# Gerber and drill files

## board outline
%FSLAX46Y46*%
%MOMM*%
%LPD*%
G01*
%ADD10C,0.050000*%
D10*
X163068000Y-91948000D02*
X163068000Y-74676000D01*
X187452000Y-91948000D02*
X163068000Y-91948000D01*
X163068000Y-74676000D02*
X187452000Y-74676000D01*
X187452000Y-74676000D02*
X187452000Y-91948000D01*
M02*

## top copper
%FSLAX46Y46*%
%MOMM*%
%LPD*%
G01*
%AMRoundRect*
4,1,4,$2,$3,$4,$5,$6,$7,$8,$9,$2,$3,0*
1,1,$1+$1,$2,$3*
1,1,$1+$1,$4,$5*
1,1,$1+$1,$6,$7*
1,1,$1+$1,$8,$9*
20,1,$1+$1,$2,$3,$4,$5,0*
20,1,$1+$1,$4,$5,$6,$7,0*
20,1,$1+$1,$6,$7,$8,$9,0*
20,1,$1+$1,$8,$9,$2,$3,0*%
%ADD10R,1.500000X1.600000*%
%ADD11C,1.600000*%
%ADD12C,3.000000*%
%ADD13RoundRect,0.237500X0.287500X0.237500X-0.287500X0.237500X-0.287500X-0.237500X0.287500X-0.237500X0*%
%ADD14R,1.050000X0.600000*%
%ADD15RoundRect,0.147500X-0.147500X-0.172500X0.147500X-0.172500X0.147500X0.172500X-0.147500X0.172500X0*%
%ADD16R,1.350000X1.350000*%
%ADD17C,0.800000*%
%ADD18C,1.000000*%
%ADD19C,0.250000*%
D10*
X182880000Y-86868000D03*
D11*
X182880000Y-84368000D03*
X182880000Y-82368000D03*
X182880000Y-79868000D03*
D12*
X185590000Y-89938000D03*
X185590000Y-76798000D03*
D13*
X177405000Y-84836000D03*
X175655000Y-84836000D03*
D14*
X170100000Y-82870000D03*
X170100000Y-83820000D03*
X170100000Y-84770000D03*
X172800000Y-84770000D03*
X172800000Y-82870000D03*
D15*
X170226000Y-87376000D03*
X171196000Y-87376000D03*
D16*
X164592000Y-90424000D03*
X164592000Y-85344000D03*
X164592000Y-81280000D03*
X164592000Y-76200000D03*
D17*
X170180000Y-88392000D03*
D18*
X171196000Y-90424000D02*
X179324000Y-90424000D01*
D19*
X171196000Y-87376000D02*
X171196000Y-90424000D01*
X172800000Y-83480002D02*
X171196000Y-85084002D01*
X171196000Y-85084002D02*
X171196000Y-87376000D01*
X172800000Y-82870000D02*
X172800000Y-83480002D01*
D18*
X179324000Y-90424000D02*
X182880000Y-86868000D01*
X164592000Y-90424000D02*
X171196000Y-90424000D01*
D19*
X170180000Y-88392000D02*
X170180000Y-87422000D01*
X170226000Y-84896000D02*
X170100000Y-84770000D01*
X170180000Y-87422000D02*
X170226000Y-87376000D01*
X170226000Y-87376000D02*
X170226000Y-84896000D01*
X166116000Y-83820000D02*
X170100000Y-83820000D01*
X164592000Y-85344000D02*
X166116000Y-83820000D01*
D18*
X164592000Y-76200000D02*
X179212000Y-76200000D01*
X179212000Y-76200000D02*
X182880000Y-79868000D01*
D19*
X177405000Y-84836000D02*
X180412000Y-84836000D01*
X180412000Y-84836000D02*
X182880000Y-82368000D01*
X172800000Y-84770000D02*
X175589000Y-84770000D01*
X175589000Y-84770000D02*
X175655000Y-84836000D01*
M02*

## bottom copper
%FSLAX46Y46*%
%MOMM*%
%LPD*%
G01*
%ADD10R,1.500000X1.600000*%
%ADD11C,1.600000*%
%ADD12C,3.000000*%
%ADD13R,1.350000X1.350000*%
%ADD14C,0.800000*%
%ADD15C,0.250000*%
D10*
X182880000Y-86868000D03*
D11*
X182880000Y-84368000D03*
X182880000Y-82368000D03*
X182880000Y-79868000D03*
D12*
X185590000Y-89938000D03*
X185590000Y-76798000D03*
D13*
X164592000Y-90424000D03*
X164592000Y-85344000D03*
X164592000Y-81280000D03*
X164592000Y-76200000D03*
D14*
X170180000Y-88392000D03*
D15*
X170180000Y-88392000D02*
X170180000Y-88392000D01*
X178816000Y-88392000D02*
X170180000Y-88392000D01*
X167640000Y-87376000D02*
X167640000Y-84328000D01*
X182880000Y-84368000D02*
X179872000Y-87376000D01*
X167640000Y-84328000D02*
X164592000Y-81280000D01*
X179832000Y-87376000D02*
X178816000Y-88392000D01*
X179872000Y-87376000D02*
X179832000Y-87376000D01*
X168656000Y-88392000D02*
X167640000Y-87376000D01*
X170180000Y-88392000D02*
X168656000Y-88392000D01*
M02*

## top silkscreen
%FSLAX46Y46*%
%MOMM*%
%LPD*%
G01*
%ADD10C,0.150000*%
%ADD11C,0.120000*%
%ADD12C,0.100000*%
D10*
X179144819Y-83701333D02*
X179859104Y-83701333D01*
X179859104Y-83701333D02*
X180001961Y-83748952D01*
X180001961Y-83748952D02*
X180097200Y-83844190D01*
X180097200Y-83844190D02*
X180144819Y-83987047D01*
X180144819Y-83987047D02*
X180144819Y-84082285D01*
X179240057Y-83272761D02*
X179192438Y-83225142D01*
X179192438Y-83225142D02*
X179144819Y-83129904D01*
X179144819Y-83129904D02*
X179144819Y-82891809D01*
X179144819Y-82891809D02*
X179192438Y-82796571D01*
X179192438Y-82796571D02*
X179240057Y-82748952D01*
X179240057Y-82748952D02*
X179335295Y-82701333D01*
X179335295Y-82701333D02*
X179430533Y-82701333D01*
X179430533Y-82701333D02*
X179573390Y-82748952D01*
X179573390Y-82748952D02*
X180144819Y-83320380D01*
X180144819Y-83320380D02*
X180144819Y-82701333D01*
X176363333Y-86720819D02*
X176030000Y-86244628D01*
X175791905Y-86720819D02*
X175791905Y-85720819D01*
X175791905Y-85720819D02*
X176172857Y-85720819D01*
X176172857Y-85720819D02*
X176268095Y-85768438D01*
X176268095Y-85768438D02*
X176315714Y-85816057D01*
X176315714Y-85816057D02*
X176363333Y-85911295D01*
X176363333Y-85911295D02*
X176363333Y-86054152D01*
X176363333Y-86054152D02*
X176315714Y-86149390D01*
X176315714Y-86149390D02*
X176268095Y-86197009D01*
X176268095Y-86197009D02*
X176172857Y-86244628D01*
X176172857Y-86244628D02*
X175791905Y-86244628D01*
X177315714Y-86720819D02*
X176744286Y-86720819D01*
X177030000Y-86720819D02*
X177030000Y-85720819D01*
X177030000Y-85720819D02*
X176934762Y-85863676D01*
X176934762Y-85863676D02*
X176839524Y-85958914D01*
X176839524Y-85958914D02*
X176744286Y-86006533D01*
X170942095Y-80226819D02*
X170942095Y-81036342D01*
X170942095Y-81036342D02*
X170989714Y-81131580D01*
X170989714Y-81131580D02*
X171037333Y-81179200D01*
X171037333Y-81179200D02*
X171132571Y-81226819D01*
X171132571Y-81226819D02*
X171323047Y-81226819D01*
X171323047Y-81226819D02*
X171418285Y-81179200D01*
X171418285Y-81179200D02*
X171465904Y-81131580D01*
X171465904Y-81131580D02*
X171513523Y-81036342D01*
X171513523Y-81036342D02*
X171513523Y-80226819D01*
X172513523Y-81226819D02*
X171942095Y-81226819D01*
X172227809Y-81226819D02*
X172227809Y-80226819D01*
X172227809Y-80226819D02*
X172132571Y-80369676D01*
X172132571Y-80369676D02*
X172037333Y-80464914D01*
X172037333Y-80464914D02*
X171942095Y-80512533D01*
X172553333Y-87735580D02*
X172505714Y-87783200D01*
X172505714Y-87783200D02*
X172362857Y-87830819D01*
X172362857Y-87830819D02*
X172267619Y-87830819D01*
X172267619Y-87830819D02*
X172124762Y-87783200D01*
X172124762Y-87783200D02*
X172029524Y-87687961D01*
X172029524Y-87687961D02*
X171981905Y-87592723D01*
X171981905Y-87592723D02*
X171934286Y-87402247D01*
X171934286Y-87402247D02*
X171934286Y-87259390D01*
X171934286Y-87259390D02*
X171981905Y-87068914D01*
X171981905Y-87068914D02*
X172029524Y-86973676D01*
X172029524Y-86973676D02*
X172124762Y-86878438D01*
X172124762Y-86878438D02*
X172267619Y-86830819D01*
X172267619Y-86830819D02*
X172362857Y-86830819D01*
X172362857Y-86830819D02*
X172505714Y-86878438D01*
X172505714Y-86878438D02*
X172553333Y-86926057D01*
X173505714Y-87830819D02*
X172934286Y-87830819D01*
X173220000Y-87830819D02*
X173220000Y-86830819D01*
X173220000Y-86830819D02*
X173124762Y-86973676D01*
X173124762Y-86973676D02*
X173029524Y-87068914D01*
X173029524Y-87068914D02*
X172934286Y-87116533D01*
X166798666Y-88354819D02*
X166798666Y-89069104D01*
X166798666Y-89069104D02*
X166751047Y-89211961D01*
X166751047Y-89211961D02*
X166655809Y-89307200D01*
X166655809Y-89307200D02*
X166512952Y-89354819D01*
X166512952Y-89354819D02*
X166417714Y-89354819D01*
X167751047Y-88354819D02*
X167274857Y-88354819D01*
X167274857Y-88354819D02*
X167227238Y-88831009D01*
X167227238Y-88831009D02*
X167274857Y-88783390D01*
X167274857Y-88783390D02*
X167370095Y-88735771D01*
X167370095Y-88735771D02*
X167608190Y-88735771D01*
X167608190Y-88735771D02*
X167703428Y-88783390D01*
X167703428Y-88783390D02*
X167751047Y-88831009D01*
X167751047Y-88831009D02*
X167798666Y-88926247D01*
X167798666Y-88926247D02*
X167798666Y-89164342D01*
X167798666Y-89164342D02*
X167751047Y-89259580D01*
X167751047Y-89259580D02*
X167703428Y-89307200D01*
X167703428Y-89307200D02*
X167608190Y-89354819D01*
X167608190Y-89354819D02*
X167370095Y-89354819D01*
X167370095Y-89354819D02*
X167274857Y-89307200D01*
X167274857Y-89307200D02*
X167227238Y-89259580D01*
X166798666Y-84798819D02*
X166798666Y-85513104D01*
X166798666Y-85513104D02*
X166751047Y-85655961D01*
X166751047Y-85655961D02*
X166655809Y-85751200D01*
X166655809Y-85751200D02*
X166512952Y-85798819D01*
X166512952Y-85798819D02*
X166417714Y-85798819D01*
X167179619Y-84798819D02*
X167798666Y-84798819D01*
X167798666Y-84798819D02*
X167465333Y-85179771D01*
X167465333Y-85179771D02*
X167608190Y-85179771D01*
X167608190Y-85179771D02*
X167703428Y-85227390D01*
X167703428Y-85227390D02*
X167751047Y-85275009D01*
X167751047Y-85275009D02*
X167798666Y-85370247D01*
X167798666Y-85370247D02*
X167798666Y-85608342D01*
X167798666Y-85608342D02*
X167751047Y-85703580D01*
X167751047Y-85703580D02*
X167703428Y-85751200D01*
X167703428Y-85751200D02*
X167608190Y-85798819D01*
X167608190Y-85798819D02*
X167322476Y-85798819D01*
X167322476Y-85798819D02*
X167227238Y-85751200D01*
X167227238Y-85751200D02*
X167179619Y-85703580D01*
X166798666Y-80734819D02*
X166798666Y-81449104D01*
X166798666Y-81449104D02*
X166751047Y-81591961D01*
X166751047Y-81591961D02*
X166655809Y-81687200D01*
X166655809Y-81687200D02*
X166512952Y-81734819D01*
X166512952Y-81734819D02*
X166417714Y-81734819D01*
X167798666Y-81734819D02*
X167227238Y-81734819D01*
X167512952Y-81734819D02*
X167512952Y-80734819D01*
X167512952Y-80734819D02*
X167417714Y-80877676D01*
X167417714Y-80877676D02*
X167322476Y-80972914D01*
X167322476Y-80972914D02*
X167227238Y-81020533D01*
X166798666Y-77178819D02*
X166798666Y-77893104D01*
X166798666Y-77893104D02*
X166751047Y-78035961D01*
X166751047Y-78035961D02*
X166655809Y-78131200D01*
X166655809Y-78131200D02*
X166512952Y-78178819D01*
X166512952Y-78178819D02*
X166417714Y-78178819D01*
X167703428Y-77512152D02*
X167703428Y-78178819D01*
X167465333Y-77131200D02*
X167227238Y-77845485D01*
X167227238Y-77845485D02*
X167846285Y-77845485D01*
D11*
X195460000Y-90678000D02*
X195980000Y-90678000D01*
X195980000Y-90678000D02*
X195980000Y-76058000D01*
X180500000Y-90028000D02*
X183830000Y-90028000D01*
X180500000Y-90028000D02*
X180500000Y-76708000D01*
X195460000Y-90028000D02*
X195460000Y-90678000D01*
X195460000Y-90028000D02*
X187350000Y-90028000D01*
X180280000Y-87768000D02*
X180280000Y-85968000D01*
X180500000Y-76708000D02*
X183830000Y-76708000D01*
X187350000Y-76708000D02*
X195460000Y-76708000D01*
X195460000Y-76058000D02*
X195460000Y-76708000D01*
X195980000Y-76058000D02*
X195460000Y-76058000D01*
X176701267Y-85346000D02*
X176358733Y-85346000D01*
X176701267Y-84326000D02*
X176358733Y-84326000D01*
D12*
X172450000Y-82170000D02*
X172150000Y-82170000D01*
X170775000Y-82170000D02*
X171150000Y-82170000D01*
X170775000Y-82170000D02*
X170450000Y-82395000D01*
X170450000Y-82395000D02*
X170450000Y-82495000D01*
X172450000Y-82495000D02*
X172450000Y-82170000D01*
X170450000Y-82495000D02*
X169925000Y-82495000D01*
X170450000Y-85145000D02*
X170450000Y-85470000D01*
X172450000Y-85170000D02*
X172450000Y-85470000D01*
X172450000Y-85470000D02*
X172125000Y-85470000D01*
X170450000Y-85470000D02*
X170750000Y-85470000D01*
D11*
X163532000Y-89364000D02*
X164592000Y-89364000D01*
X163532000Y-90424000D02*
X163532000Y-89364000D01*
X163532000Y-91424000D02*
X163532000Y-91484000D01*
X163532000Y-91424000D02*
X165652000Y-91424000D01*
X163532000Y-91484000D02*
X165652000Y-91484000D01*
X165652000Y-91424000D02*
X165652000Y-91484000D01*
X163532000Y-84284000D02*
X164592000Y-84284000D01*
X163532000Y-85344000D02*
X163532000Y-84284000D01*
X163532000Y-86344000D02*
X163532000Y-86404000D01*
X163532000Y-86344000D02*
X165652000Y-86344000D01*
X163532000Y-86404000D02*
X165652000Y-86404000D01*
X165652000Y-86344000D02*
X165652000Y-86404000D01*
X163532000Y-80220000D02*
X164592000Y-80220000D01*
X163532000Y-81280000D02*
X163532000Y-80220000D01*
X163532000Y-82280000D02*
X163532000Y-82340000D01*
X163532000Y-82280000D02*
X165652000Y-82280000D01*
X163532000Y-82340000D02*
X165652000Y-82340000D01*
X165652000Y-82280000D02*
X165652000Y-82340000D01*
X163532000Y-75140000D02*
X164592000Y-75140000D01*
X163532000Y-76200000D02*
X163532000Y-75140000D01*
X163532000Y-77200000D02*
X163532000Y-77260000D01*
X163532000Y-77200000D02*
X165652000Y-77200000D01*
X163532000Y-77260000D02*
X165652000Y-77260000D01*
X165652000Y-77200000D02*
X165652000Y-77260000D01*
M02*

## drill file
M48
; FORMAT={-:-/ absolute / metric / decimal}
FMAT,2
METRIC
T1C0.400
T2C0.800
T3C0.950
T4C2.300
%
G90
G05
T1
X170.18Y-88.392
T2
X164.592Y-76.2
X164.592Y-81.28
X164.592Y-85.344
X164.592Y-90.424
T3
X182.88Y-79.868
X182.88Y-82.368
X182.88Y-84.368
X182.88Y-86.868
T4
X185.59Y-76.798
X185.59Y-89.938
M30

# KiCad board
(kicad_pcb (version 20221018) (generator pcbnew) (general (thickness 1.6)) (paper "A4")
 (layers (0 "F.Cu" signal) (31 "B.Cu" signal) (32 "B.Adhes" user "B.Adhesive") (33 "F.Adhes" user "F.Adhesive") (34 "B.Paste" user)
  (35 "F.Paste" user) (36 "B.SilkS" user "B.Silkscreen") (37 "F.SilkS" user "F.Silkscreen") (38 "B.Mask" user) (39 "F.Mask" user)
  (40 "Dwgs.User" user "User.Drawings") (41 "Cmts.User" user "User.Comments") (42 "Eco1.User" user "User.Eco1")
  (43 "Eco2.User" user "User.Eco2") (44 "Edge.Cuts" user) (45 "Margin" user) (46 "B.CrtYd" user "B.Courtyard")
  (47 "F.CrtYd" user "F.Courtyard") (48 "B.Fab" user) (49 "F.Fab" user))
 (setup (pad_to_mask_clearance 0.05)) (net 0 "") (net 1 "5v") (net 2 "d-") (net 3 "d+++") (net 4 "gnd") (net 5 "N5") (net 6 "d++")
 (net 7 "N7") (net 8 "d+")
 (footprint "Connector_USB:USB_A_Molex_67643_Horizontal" (layer "F.Cu") (at 182.88 86.868 90)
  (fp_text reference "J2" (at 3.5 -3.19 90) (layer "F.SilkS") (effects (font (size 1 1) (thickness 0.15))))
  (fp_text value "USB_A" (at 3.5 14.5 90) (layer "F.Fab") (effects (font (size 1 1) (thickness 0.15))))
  (fp_line (start -3.81 12.58) (end -3.81 13.1) (stroke (width 0.12) (type solid)) (layer "F.SilkS"))
  (fp_line (start -3.81 13.1) (end 10.81 13.1) (stroke (width 0.12) (type solid)) (layer "F.SilkS"))
  (fp_line (start -3.16 -2.38) (end -3.16 0.95) (stroke (width 0.12) (type solid)) (layer "F.SilkS"))
  (fp_line (start -3.16 -2.38) (end 10.16 -2.38) (stroke (width 0.12) (type solid)) (layer "F.SilkS"))
  (fp_line (start -3.16 12.58) (end -3.81 12.58) (stroke (width 0.12) (type solid)) (layer "F.SilkS"))
  (fp_line (start -3.16 12.58) (end -3.16 4.47) (stroke (width 0.12) (type solid)) (layer "F.SilkS"))
  (fp_line (start -0.9 -2.6) (end 0.9 -2.6) (stroke (width 0.12) (type solid)) (layer "F.SilkS"))
  (fp_line (start 10.16 -2.38) (end 10.16 0.95) (stroke (width 0.12) (type solid)) (layer "F.SilkS"))
  (fp_line (start 10.16 4.47) (end 10.16 12.58) (stroke (width 0.12) (type solid)) (layer "F.SilkS"))
  (fp_line (start 10.81 12.58) (end 10.16 12.58) (stroke (width 0.12) (type solid)) (layer "F.SilkS"))
  (fp_line (start 10.81 13.1) (end 10.81 12.58) (stroke (width 0.12) (type solid)) (layer "F.SilkS"))
  (pad "1" thru_hole rect (at 0 0 90) (size 1.6 1.5) (drill 0.95) (layers "*.Cu" "*.Mask") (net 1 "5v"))
  (pad "2" thru_hole circle (at 2.5 0 90) (size 1.6 1.6) (drill 0.95) (layers "*.Cu" "*.Mask") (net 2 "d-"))
  (pad "3" thru_hole circle (at 4.5 0 90) (size 1.6 1.6) (drill 0.95) (layers "*.Cu" "*.Mask") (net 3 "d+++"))
  (pad "4" thru_hole circle (at 7 0 90) (size 1.6 1.6) (drill 0.95) (layers "*.Cu" "*.Mask") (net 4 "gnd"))
  (pad "5" thru_hole circle (at -3.07 2.71 90) (size 3 3) (drill 2.3) (layers "*.Cu" "*.Mask") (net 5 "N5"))
  (pad "5" thru_hole circle (at 10.07 2.71 90) (size 3 3) (drill 2.3) (layers "*.Cu" "*.Mask") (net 5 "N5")))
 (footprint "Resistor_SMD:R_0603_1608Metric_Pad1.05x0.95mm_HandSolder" (layer "F.Cu") (at 176.53 84.836 180)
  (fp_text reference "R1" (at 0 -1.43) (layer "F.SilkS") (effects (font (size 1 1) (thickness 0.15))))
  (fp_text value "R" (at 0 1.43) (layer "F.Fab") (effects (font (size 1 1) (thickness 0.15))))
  (fp_line (start -0.171267 -0.51) (end 0.171267 -0.51) (stroke (width 0.12) (type solid)) (layer "F.SilkS"))
  (fp_line (start -0.171267 0.51) (end 0.171267 0.51) (stroke (width 0.12) (type solid)) (layer "F.SilkS"))
  (pad "1" smd roundrect (at -0.875 0 180) (size 1.05 0.95) (layers "F.Cu" "F.Paste" "F.Mask") (roundrect_rratio 0.25) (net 3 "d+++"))
  (pad "2" smd roundrect (at 0.875 0 180) (size 1.05 0.95) (layers "F.Cu" "F.Paste" "F.Mask") (roundrect_rratio 0.25) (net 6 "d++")))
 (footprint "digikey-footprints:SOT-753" (layer "F.Cu") (at 171.45 83.82 -90)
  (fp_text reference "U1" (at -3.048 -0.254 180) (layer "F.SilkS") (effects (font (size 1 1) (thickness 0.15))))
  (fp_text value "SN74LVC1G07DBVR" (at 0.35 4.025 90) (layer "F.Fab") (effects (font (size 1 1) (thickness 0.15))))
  (fp_line (start -1.65 -1) (end -1.65 -0.7) (stroke (width 0.1) (type solid)) (layer "F.SilkS"))
  (fp_line (start -1.65 0.675) (end -1.65 0.3) (stroke (width 0.1) (type solid)) (layer "F.SilkS"))
  (fp_line (start -1.65 0.675) (end -1.425 1) (stroke (width 0.1) (type solid)) (layer "F.SilkS"))
  (fp_line (start -1.425 1) (end -1.325 1) (stroke (width 0.1) (type solid)) (layer "F.SilkS"))
  (fp_line (start -1.325 -1) (end -1.65 -1) (stroke (width 0.1) (type solid)) (layer "F.SilkS"))
  (fp_line (start -1.325 1) (end -1.325 1.525) (stroke (width 0.1) (type solid)) (layer "F.SilkS"))
  (fp_line (start 1.325 1) (end 1.65 1) (stroke (width 0.1) (type solid)) (layer "F.SilkS"))
  (fp_line (start 1.35 -1) (end 1.65 -1) (stroke (width 0.1) (type solid)) (layer "F.SilkS"))
  (fp_line (start 1.65 -1) (end 1.65 -0.675) (stroke (width 0.1) (type solid)) (layer "F.SilkS"))
  (fp_line (start 1.65 1) (end 1.65 0.7) (stroke (width 0.1) (type solid)) (layer "F.SilkS"))
  (pad "1" smd rect (at -0.95 1.35 270) (size 0.6 1.05) (layers "F.Cu" "F.Paste" "F.Mask") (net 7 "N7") (solder_mask_margin 0.07))
  (pad "2" smd rect (at 0 1.35 270) (size 0.6 1.05) (layers "F.Cu" "F.Paste" "F.Mask") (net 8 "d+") (solder_mask_margin 0.07))
  (pad "3" smd rect (at 0.95 1.35 270) (size 0.6 1.05) (layers "F.Cu" "F.Paste" "F.Mask") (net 2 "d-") (solder_mask_margin 0.07))
  (pad "4" smd rect (at 0.95 -1.35 270) (size 0.6 1.05) (layers "F.Cu" "F.Paste" "F.Mask") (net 6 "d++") (solder_mask_margin 0.07))
  (pad "5" smd rect (at -0.95 -1.35 270) (size 0.6 1.05) (layers "F.Cu" "F.Paste" "F.Mask") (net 1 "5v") (solder_mask_margin 0.07)))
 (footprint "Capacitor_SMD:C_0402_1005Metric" (layer "F.Cu") (at 170.711 87.376)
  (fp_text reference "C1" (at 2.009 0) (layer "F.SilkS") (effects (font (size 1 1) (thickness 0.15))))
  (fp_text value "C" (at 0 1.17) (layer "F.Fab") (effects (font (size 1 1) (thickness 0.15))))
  (pad "1" smd roundrect (at -0.485 0) (size 0.59 0.64) (layers "F.Cu" "F.Paste" "F.Mask") (roundrect_rratio 0.25) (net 2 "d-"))
  (pad "2" smd roundrect (at 0.485 0) (size 0.59 0.64) (layers "F.Cu" "F.Paste" "F.Mask") (roundrect_rratio 0.25) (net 1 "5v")))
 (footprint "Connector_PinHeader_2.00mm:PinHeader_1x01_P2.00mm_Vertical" (layer "F.Cu") (at 164.592 90.424)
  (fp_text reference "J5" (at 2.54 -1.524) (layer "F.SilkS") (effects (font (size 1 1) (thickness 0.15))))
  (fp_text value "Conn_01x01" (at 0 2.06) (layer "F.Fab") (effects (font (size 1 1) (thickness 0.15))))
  (fp_line (start -1.06 -1.06) (end 0 -1.06) (stroke (width 0.12) (type solid)) (layer "F.SilkS"))
  (fp_line (start -1.06 0) (end -1.06 -1.06) (stroke (width 0.12) (type solid)) (layer "F.SilkS"))
  (fp_line (start -1.06 1) (end -1.06 1.06) (stroke (width 0.12) (type solid)) (layer "F.SilkS"))
  (fp_line (start -1.06 1) (end 1.06 1) (stroke (width 0.12) (type solid)) (layer "F.SilkS"))
  (fp_line (start -1.06 1.06) (end 1.06 1.06) (stroke (width 0.12) (type solid)) (layer "F.SilkS"))
  (fp_line (start 1.06 1) (end 1.06 1.06) (stroke (width 0.12) (type solid)) (layer "F.SilkS"))
  (pad "1" thru_hole rect (at 0 0) (size 1.35 1.35) (drill 0.8) (layers "*.Cu" "*.Mask") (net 1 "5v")))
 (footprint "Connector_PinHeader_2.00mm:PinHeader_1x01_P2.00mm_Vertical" (layer "F.Cu") (at 164.592 85.344)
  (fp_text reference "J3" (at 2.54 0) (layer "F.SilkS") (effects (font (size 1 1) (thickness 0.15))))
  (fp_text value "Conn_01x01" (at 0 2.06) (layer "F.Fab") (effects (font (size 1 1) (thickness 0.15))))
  (fp_line (start -1.06 -1.06) (end 0 -1.06) (stroke (width 0.12) (type solid)) (layer "F.SilkS"))
  (fp_line (start -1.06 0) (end -1.06 -1.06) (stroke (width 0.12) (type solid)) (layer "F.SilkS"))
  (fp_line (start -1.06 1) (end -1.06 1.06) (stroke (width 0.12) (type solid)) (layer "F.SilkS"))
  (fp_line (start -1.06 1) (end 1.06 1) (stroke (width 0.12) (type solid)) (layer "F.SilkS"))
  (fp_line (start -1.06 1.06) (end 1.06 1.06) (stroke (width 0.12) (type solid)) (layer "F.SilkS"))
  (fp_line (start 1.06 1) (end 1.06 1.06) (stroke (width 0.12) (type solid)) (layer "F.SilkS"))
  (pad "1" thru_hole rect (at 0 0) (size 1.35 1.35) (drill 0.8) (layers "*.Cu" "*.Mask") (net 8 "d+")))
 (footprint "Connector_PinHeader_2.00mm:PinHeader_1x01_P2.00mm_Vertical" (layer "F.Cu") (at 164.592 81.28)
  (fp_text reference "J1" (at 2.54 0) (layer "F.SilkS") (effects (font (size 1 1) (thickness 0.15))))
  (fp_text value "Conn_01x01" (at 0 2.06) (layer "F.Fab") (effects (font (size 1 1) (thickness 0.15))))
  (fp_line (start -1.06 -1.06) (end 0 -1.06) (stroke (width 0.12) (type solid)) (layer "F.SilkS"))
  (fp_line (start -1.06 0) (end -1.06 -1.06) (stroke (width 0.12) (type solid)) (layer "F.SilkS"))
  (fp_line (start -1.06 1) (end -1.06 1.06) (stroke (width 0.12) (type solid)) (layer "F.SilkS"))
  (fp_line (start -1.06 1) (end 1.06 1) (stroke (width 0.12) (type solid)) (layer "F.SilkS"))
  (fp_line (start -1.06 1.06) (end 1.06 1.06) (stroke (width 0.12) (type solid)) (layer "F.SilkS"))
  (fp_line (start 1.06 1) (end 1.06 1.06) (stroke (width 0.12) (type solid)) (layer "F.SilkS"))
  (pad "1" thru_hole rect (at 0 0) (size 1.35 1.35) (drill 0.8) (layers "*.Cu" "*.Mask") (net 2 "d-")))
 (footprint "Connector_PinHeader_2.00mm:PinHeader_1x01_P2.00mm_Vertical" (layer "F.Cu") (at 164.592 76.2)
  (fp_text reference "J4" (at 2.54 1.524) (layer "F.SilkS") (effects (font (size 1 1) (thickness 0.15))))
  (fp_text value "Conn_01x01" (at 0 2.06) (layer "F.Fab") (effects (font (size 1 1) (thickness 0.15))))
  (fp_line (start -1.06 -1.06) (end 0 -1.06) (stroke (width 0.12) (type solid)) (layer "F.SilkS"))
  (fp_line (start -1.06 0) (end -1.06 -1.06) (stroke (width 0.12) (type solid)) (layer "F.SilkS"))
  (fp_line (start -1.06 1) (end -1.06 1.06) (stroke (width 0.12) (type solid)) (layer "F.SilkS"))
  (fp_line (start -1.06 1) (end 1.06 1) (stroke (width 0.12) (type solid)) (layer "F.SilkS"))
  (fp_line (start -1.06 1.06) (end 1.06 1.06) (stroke (width 0.12) (type solid)) (layer "F.SilkS"))
  (fp_line (start 1.06 1) (end 1.06 1.06) (stroke (width 0.12) (type solid)) (layer "F.SilkS"))
  (pad "1" thru_hole rect (at 0 0) (size 1.35 1.35) (drill 0.8) (layers "*.Cu" "*.Mask") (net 4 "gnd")))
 (gr_line (start 163.068 91.948) (end 163.068 74.676) (stroke (width 0.05) (type solid)) (layer "Edge.Cuts"))
 (gr_line (start 187.452 91.948) (end 163.068 91.948) (stroke (width 0.05) (type solid)) (layer "Edge.Cuts"))
 (gr_line (start 163.068 74.676) (end 187.452 74.676) (stroke (width 0.05) (type solid)) (layer "Edge.Cuts"))
 (gr_line (start 187.452 74.676) (end 187.452 91.948) (stroke (width 0.05) (type solid)) (layer "Edge.Cuts"))
 (segment (start 171.196 90.424) (end 179.324 90.424) (width 1) (layer "F.Cu") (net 1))
 (segment (start 171.196 87.376) (end 171.196 90.424) (width 0.25) (layer "F.Cu") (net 1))
 (segment (start 172.8 83.480002) (end 171.196 85.084002) (width 0.25) (layer "F.Cu") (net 1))
 (segment (start 171.196 85.084002) (end 171.196 87.376) (width 0.25) (layer "F.Cu") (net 1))
 (segment (start 172.8 82.87) (end 172.8 83.480002) (width 0.25) (layer "F.Cu") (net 1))
 (segment (start 179.324 90.424) (end 182.88 86.868) (width 1) (layer "F.Cu") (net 1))
 (segment (start 164.592 90.424) (end 171.196 90.424) (width 1) (layer "F.Cu") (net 1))
 (segment (start 170.18 88.392) (end 170.18 87.422) (width 0.25) (layer "F.Cu") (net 2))
 (segment (start 170.226 84.896) (end 170.1 84.77) (width 0.25) (layer "F.Cu") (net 2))
 (segment (start 170.18 87.422) (end 170.226 87.376) (width 0.25) (layer "F.Cu") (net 2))
 (segment (start 170.226 87.376) (end 170.226 84.896) (width 0.25) (layer "F.Cu") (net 2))
 (via (at 170.18 88.392) (size 0.8) (drill 0.4) (layers "F.Cu" "B.Cu") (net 2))
 (segment (start 170.18 88.392) (end 170.18 88.392) (width 0.25) (layer "B.Cu") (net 2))
 (segment (start 178.816 88.392) (end 170.18 88.392) (width 0.25) (layer "B.Cu") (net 2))
 (segment (start 167.64 87.376) (end 167.64 84.328) (width 0.25) (layer "B.Cu") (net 2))
 (segment (start 182.88 84.368) (end 179.872 87.376) (width 0.25) (layer "B.Cu") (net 2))
 (segment (start 167.64 84.328) (end 164.592 81.28) (width 0.25) (layer "B.Cu") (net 2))
 (segment (start 179.832 87.376) (end 178.816 88.392) (width 0.25) (layer "B.Cu") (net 2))
 (segment (start 179.872 87.376) (end 179.832 87.376) (width 0.25) (layer "B.Cu") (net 2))
 (segment (start 168.656 88.392) (end 167.64 87.376) (width 0.25) (layer "B.Cu") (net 2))
 (segment (start 170.18 88.392) (end 168.656 88.392) (width 0.25) (layer "B.Cu") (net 2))
 (segment (start 166.116 83.82) (end 170.1 83.82) (width 0.25) (layer "F.Cu") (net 8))
 (segment (start 164.592 85.344) (end 166.116 83.82) (width 0.25) (layer "F.Cu") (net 8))
 (segment (start 164.592 76.2) (end 179.212 76.2) (width 1) (layer "F.Cu") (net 4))
 (segment (start 179.212 76.2) (end 182.88 79.868) (width 1) (layer "F.Cu") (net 4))
 (segment (start 177.405 84.836) (end 180.412 84.836) (width 0.25) (layer "F.Cu") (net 3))
 (segment (start 180.412 84.836) (end 182.88 82.368) (width 0.25) (layer "F.Cu") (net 3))
 (segment (start 172.8 84.77) (end 175.589 84.77) (width 0.25) (layer "F.Cu") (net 6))
 (segment (start 175.589 84.77) (end 175.655 84.836) (width 0.25) (layer "F.Cu") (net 6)))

